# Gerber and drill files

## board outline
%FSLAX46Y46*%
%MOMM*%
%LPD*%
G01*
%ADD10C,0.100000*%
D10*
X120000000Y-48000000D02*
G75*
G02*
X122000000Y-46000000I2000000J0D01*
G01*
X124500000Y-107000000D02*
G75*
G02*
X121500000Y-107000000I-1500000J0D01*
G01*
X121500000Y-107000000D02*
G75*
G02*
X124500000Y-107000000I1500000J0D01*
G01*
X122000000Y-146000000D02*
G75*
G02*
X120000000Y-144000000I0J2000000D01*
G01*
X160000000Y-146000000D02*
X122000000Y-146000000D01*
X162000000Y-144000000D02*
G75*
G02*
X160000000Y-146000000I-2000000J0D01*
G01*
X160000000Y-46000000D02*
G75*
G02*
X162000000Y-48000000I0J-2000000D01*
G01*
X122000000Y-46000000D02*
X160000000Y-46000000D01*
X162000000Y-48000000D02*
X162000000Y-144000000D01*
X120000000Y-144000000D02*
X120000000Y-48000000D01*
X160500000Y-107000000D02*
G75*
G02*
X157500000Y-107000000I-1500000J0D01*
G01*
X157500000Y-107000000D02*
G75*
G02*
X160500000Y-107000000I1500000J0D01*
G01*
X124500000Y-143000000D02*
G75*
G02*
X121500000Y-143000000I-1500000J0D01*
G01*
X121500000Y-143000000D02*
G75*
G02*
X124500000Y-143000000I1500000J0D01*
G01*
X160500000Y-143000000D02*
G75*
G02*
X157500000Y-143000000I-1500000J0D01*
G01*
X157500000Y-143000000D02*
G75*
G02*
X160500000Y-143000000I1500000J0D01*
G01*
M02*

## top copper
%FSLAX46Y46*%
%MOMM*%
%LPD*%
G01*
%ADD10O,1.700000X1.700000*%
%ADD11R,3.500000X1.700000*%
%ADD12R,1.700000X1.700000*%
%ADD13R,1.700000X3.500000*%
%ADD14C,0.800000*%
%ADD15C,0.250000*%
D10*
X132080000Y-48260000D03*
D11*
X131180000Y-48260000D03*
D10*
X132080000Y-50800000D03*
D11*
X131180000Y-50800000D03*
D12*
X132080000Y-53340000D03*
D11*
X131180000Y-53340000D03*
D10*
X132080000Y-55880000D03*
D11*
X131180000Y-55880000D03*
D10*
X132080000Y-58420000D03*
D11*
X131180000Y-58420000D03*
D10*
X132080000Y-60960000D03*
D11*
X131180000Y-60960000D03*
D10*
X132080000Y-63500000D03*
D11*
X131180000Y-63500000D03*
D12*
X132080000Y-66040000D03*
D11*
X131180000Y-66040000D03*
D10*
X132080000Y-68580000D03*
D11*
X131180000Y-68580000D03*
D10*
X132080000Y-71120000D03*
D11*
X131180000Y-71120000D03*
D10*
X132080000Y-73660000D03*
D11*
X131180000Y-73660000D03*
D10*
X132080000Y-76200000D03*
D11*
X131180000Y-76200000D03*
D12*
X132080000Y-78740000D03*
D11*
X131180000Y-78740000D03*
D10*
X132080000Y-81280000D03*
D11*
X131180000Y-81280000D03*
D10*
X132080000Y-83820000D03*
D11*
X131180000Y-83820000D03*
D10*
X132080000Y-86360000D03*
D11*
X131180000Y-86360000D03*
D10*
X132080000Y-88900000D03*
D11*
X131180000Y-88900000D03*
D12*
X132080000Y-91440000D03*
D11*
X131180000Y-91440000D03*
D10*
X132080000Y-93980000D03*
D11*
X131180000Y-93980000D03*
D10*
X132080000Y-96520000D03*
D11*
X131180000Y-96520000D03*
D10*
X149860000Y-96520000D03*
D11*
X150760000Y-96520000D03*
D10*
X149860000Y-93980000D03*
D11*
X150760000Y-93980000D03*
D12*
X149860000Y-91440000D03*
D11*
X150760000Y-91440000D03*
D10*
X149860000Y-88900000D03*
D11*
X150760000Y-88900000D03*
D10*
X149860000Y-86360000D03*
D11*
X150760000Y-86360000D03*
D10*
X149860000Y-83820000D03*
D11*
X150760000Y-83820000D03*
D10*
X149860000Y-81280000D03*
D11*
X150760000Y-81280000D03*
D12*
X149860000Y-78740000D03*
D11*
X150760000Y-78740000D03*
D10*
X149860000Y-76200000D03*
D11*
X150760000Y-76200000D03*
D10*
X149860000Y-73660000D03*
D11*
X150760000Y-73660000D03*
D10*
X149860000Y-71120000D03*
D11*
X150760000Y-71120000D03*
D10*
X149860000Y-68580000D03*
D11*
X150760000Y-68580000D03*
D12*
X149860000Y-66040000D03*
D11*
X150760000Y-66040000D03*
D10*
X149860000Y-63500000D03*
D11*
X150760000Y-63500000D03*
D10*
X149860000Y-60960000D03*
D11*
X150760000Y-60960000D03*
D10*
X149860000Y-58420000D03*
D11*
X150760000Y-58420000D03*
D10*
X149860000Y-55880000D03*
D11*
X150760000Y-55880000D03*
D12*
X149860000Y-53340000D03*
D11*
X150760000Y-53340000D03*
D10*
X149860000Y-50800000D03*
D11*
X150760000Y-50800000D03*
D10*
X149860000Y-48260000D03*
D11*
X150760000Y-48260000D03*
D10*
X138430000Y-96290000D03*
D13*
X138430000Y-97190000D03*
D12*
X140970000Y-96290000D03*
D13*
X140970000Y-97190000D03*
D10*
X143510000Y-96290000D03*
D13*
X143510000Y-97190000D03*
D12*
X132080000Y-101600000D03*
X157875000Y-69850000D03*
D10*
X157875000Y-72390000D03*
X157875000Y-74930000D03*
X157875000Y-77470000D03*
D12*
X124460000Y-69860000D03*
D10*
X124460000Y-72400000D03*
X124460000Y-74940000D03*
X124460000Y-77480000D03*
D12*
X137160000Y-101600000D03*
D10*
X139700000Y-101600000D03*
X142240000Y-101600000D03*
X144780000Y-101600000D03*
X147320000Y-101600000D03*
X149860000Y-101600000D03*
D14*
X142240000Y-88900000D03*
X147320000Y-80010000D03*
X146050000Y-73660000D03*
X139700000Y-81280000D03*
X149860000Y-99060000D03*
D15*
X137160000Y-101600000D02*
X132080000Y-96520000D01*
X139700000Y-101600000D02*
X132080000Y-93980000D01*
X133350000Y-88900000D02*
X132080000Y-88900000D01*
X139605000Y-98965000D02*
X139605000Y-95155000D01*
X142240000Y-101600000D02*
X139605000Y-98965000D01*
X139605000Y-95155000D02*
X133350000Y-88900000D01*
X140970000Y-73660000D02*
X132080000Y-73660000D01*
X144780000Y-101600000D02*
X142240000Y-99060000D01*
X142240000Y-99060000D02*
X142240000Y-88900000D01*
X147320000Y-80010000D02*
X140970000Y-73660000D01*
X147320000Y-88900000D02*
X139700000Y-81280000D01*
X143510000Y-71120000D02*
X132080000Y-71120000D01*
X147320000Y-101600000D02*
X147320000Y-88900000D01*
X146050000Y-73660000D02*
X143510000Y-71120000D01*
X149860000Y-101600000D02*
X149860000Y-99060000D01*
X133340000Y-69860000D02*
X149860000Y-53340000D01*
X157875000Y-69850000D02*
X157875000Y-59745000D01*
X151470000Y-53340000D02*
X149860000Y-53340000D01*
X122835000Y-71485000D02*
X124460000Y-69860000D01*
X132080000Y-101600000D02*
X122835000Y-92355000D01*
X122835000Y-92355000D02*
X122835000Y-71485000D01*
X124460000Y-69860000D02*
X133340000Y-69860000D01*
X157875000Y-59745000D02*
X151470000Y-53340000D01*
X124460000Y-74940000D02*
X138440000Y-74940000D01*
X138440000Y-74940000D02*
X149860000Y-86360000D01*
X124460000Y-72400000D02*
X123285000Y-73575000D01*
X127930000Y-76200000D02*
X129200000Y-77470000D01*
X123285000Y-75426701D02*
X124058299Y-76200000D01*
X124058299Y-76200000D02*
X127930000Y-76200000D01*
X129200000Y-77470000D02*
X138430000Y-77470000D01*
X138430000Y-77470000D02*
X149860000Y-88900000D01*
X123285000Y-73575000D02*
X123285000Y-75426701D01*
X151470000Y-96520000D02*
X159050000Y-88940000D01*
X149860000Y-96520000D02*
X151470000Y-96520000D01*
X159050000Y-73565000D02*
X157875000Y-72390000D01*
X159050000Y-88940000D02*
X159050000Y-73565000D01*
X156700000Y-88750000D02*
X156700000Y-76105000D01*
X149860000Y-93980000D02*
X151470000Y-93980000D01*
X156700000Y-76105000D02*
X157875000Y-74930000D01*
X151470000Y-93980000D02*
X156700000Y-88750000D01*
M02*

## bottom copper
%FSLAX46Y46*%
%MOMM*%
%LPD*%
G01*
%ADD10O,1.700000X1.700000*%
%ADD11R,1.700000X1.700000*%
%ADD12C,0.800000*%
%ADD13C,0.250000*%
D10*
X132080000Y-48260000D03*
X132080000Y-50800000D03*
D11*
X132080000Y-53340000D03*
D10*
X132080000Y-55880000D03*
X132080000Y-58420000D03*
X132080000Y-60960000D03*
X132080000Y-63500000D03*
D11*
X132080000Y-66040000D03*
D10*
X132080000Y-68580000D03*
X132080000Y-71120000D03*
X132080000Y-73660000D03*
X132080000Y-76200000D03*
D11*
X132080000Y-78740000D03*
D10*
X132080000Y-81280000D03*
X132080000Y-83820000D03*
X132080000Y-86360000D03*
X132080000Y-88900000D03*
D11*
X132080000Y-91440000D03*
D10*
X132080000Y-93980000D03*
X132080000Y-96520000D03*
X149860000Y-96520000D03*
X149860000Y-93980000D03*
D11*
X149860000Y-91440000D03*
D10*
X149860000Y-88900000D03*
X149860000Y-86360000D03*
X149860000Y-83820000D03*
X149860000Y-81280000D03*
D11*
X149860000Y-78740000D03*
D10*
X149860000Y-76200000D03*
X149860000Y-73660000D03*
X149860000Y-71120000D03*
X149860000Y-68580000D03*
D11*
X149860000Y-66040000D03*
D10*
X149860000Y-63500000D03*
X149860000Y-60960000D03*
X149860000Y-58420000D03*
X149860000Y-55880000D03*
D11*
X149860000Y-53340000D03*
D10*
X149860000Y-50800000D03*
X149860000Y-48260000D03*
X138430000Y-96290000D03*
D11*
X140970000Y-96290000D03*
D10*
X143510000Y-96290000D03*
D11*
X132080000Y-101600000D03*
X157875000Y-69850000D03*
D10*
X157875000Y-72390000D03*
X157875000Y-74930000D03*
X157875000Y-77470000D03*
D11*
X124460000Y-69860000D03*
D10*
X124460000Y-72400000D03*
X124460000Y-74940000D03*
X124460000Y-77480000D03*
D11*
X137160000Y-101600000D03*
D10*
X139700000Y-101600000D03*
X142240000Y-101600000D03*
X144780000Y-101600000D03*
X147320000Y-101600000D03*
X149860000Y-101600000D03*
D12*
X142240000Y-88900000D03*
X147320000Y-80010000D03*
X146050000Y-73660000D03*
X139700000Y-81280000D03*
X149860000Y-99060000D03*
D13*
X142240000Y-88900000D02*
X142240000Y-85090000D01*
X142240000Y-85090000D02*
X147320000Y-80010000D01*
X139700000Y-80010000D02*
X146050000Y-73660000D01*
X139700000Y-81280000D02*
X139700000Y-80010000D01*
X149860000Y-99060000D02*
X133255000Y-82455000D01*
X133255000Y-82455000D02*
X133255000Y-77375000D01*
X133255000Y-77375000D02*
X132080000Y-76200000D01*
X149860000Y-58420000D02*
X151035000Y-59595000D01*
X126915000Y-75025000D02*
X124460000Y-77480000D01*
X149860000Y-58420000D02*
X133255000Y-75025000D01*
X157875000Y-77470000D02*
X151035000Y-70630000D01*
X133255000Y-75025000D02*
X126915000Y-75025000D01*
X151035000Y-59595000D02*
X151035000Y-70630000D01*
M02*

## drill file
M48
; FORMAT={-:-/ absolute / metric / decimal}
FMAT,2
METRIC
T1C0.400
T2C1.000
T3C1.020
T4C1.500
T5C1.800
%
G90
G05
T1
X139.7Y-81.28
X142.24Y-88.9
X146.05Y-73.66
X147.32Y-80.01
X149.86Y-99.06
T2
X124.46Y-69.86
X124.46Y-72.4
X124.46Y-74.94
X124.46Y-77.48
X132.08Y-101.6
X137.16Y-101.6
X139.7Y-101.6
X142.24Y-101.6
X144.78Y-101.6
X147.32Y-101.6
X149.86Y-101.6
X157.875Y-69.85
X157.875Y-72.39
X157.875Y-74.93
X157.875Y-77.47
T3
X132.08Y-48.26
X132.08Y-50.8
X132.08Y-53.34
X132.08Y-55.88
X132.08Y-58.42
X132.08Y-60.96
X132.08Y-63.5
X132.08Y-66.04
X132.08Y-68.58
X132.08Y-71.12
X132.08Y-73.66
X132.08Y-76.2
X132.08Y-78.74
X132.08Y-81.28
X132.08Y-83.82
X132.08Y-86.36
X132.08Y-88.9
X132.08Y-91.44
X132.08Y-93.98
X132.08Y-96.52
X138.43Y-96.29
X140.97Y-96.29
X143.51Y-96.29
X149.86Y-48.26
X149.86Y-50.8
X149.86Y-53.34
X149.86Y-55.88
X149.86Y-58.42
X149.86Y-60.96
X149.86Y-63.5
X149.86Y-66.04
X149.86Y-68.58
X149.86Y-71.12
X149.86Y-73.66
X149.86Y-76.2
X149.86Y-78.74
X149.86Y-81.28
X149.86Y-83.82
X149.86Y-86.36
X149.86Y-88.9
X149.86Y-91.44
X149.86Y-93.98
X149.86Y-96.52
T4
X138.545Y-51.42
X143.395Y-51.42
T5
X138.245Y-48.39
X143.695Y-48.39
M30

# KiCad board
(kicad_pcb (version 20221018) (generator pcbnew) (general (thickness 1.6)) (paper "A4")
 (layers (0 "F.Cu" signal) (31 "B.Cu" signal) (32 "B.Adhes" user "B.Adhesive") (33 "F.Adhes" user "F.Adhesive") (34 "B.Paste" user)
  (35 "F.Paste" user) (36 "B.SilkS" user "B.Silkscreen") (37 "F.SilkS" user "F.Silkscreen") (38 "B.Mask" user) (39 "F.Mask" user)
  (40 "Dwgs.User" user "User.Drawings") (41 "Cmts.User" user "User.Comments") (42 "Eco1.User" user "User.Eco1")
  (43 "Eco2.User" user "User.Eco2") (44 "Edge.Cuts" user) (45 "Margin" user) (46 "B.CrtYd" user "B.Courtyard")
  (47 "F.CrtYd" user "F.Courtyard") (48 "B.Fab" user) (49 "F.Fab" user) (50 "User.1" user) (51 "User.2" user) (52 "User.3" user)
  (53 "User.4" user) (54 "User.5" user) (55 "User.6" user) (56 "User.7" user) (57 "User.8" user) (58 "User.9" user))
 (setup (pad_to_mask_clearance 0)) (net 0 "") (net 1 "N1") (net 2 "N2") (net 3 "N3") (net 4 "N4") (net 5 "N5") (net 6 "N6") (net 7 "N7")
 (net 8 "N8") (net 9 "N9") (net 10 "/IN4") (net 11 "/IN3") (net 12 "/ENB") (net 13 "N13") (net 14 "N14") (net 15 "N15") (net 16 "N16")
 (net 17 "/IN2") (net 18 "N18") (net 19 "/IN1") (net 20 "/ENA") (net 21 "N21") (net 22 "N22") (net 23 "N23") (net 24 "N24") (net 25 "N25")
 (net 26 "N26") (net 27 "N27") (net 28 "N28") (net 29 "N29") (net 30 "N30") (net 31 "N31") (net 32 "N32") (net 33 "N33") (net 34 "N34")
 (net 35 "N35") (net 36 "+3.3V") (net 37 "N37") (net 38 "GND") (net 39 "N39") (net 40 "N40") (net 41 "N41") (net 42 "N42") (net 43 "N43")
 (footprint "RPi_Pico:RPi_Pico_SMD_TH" (layer "F.Cu") (at 140.97 72.39)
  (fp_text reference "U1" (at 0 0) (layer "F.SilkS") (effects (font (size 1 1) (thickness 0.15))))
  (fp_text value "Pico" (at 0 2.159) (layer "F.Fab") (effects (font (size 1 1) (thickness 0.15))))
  (pad "" np_thru_hole oval (at -2.725 -24) (size 1.8 1.8) (drill 1.8) (layers "*.Cu" "*.Mask"))
  (pad "" np_thru_hole oval (at -2.425 -20.97) (size 1.5 1.5) (drill 1.5) (layers "*.Cu" "*.Mask"))
  (pad "" np_thru_hole oval (at 2.425 -20.97) (size 1.5 1.5) (drill 1.5) (layers "*.Cu" "*.Mask"))
  (pad "" np_thru_hole oval (at 2.725 -24) (size 1.8 1.8) (drill 1.8) (layers "*.Cu" "*.Mask"))
  (pad "1" thru_hole oval (at -8.89 -24.13) (size 1.7 1.7) (drill 1.02) (layers "*.Cu" "*.Mask") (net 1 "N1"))
  (pad "1" smd rect (at -8.89 -24.13) (size 3.5 1.7) (drill (offset -0.9 0)) (layers "F.Cu" "F.Mask") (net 1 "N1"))
  (pad "2" thru_hole oval (at -8.89 -21.59) (size 1.7 1.7) (drill 1.02) (layers "*.Cu" "*.Mask") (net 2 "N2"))
  (pad "2" smd rect (at -8.89 -21.59) (size 3.5 1.7) (drill (offset -0.9 0)) (layers "F.Cu" "F.Mask") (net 2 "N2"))
  (pad "3" thru_hole rect (at -8.89 -19.05) (size 1.7 1.7) (drill 1.02) (layers "*.Cu" "*.Mask") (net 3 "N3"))
  (pad "3" smd rect (at -8.89 -19.05) (size 3.5 1.7) (drill (offset -0.9 0)) (layers "F.Cu" "F.Mask") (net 3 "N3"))
  (pad "4" thru_hole oval (at -8.89 -16.51) (size 1.7 1.7) (drill 1.02) (layers "*.Cu" "*.Mask") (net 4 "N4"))
  (pad "4" smd rect (at -8.89 -16.51) (size 3.5 1.7) (drill (offset -0.9 0)) (layers "F.Cu" "F.Mask") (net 4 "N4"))
  (pad "5" thru_hole oval (at -8.89 -13.97) (size 1.7 1.7) (drill 1.02) (layers "*.Cu" "*.Mask") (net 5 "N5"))
  (pad "5" smd rect (at -8.89 -13.97) (size 3.5 1.7) (drill (offset -0.9 0)) (layers "F.Cu" "F.Mask") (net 5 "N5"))
  (pad "6" thru_hole oval (at -8.89 -11.43) (size 1.7 1.7) (drill 1.02) (layers "*.Cu" "*.Mask") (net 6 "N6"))
  (pad "6" smd rect (at -8.89 -11.43) (size 3.5 1.7) (drill (offset -0.9 0)) (layers "F.Cu" "F.Mask") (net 6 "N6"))
  (pad "7" thru_hole oval (at -8.89 -8.89) (size 1.7 1.7) (drill 1.02) (layers "*.Cu" "*.Mask") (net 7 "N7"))
  (pad "7" smd rect (at -8.89 -8.89) (size 3.5 1.7) (drill (offset -0.9 0)) (layers "F.Cu" "F.Mask") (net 7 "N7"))
  (pad "8" thru_hole rect (at -8.89 -6.35) (size 1.7 1.7) (drill 1.02) (layers "*.Cu" "*.Mask") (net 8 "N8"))
  (pad "8" smd rect (at -8.89 -6.35) (size 3.5 1.7) (drill (offset -0.9 0)) (layers "F.Cu" "F.Mask") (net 8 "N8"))
  (pad "9" thru_hole oval (at -8.89 -3.81) (size 1.7 1.7) (drill 1.02) (layers "*.Cu" "*.Mask") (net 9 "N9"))
  (pad "9" smd rect (at -8.89 -3.81) (size 3.5 1.7) (drill (offset -0.9 0)) (layers "F.Cu" "F.Mask") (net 9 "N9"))
  (pad "10" thru_hole oval (at -8.89 -1.27) (size 1.7 1.7) (drill 1.02) (layers "*.Cu" "*.Mask") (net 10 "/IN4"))
  (pad "10" smd rect (at -8.89 -1.27) (size 3.5 1.7) (drill (offset -0.9 0)) (layers "F.Cu" "F.Mask") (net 10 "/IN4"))
  (pad "11" thru_hole oval (at -8.89 1.27) (size 1.7 1.7) (drill 1.02) (layers "*.Cu" "*.Mask") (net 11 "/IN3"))
  (pad "11" smd rect (at -8.89 1.27) (size 3.5 1.7) (drill (offset -0.9 0)) (layers "F.Cu" "F.Mask") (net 11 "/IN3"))
  (pad "12" thru_hole oval (at -8.89 3.81) (size 1.7 1.7) (drill 1.02) (layers "*.Cu" "*.Mask") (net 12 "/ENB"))
  (pad "12" smd rect (at -8.89 3.81) (size 3.5 1.7) (drill (offset -0.9 0)) (layers "F.Cu" "F.Mask") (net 12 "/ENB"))
  (pad "13" thru_hole rect (at -8.89 6.35) (size 1.7 1.7) (drill 1.02) (layers "*.Cu" "*.Mask") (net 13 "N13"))
  (pad "13" smd rect (at -8.89 6.35) (size 3.5 1.7) (drill (offset -0.9 0)) (layers "F.Cu" "F.Mask") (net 13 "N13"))
  (pad "14" thru_hole oval (at -8.89 8.89) (size 1.7 1.7) (drill 1.02) (layers "*.Cu" "*.Mask") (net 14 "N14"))
  (pad "14" smd rect (at -8.89 8.89) (size 3.5 1.7) (drill (offset -0.9 0)) (layers "F.Cu" "F.Mask") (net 14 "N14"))
  (pad "15" thru_hole oval (at -8.89 11.43) (size 1.7 1.7) (drill 1.02) (layers "*.Cu" "*.Mask") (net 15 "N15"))
  (pad "15" smd rect (at -8.89 11.43) (size 3.5 1.7) (drill (offset -0.9 0)) (layers "F.Cu" "F.Mask") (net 15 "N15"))
  (pad "16" thru_hole oval (at -8.89 13.97) (size 1.7 1.7) (drill 1.02) (layers "*.Cu" "*.Mask") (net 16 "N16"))
  (pad "16" smd rect (at -8.89 13.97) (size 3.5 1.7) (drill (offset -0.9 0)) (layers "F.Cu" "F.Mask") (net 16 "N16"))
  (pad "17" thru_hole oval (at -8.89 16.51) (size 1.7 1.7) (drill 1.02) (layers "*.Cu" "*.Mask") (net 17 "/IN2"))
  (pad "17" smd rect (at -8.89 16.51) (size 3.5 1.7) (drill (offset -0.9 0)) (layers "F.Cu" "F.Mask") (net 17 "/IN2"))
  (pad "18" thru_hole rect (at -8.89 19.05) (size 1.7 1.7) (drill 1.02) (layers "*.Cu" "*.Mask") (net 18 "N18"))
  (pad "18" smd rect (at -8.89 19.05) (size 3.5 1.7) (drill (offset -0.9 0)) (layers "F.Cu" "F.Mask") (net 18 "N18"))
  (pad "19" thru_hole oval (at -8.89 21.59) (size 1.7 1.7) (drill 1.02) (layers "*.Cu" "*.Mask") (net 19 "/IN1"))
  (pad "19" smd rect (at -8.89 21.59) (size 3.5 1.7) (drill (offset -0.9 0)) (layers "F.Cu" "F.Mask") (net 19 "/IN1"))
  (pad "20" thru_hole oval (at -8.89 24.13) (size 1.7 1.7) (drill 1.02) (layers "*.Cu" "*.Mask") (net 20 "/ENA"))
  (pad "20" smd rect (at -8.89 24.13) (size 3.5 1.7) (drill (offset -0.9 0)) (layers "F.Cu" "F.Mask") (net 20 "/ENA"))
  (pad "21" thru_hole oval (at 8.89 24.13) (size 1.7 1.7) (drill 1.02) (layers "*.Cu" "*.Mask") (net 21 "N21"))
  (pad "21" smd rect (at 8.89 24.13) (size 3.5 1.7) (drill (offset 0.9 0)) (layers "F.Cu" "F.Mask") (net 21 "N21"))
  (pad "22" thru_hole oval (at 8.89 21.59) (size 1.7 1.7) (drill 1.02) (layers "*.Cu" "*.Mask") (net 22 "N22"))
  (pad "22" smd rect (at 8.89 21.59) (size 3.5 1.7) (drill (offset 0.9 0)) (layers "F.Cu" "F.Mask") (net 22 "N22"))
  (pad "23" thru_hole rect (at 8.89 19.05) (size 1.7 1.7) (drill 1.02) (layers "*.Cu" "*.Mask") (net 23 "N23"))
  (pad "23" smd rect (at 8.89 19.05) (size 3.5 1.7) (drill (offset 0.9 0)) (layers "F.Cu" "F.Mask") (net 23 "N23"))
  (pad "24" thru_hole oval (at 8.89 16.51) (size 1.7 1.7) (drill 1.02) (layers "*.Cu" "*.Mask") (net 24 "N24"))
  (pad "24" smd rect (at 8.89 16.51) (size 3.5 1.7) (drill (offset 0.9 0)) (layers "F.Cu" "F.Mask") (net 24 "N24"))
  (pad "25" thru_hole oval (at 8.89 13.97) (size 1.7 1.7) (drill 1.02) (layers "*.Cu" "*.Mask") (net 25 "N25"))
  (pad "25" smd rect (at 8.89 13.97) (size 3.5 1.7) (drill (offset 0.9 0)) (layers "F.Cu" "F.Mask") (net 25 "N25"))
  (pad "26" thru_hole oval (at 8.89 11.43) (size 1.7 1.7) (drill 1.02) (layers "*.Cu" "*.Mask") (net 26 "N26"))
  (pad "26" smd rect (at 8.89 11.43) (size 3.5 1.7) (drill (offset 0.9 0)) (layers "F.Cu" "F.Mask") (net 26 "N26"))
  (pad "27" thru_hole oval (at 8.89 8.89) (size 1.7 1.7) (drill 1.02) (layers "*.Cu" "*.Mask") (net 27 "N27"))
  (pad "27" smd rect (at 8.89 8.89) (size 3.5 1.7) (drill (offset 0.9 0)) (layers "F.Cu" "F.Mask") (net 27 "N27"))
  (pad "28" thru_hole rect (at 8.89 6.35) (size 1.7 1.7) (drill 1.02) (layers "*.Cu" "*.Mask") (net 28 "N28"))
  (pad "28" smd rect (at 8.89 6.35) (size 3.5 1.7) (drill (offset 0.9 0)) (layers "F.Cu" "F.Mask") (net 28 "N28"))
  (pad "29" thru_hole oval (at 8.89 3.81) (size 1.7 1.7) (drill 1.02) (layers "*.Cu" "*.Mask") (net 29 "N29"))
  (pad "29" smd rect (at 8.89 3.81) (size 3.5 1.7) (drill (offset 0.9 0)) (layers "F.Cu" "F.Mask") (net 29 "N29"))
  (pad "30" thru_hole oval (at 8.89 1.27) (size 1.7 1.7) (drill 1.02) (layers "*.Cu" "*.Mask") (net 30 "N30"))
  (pad "30" smd rect (at 8.89 1.27) (size 3.5 1.7) (drill (offset 0.9 0)) (layers "F.Cu" "F.Mask") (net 30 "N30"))
  (pad "31" thru_hole oval (at 8.89 -1.27) (size 1.7 1.7) (drill 1.02) (layers "*.Cu" "*.Mask") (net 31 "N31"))
  (pad "31" smd rect (at 8.89 -1.27) (size 3.5 1.7) (drill (offset 0.9 0)) (layers "F.Cu" "F.Mask") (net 31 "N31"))
  (pad "32" thru_hole oval (at 8.89 -3.81) (size 1.7 1.7) (drill 1.02) (layers "*.Cu" "*.Mask") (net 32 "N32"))
  (pad "32" smd rect (at 8.89 -3.81) (size 3.5 1.7) (drill (offset 0.9 0)) (layers "F.Cu" "F.Mask") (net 32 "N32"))
  (pad "33" thru_hole rect (at 8.89 -6.35) (size 1.7 1.7) (drill 1.02) (layers "*.Cu" "*.Mask") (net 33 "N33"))
  (pad "33" smd rect (at 8.89 -6.35) (size 3.5 1.7) (drill (offset 0.9 0)) (layers "F.Cu" "F.Mask") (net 33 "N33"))
  (pad "34" thru_hole oval (at 8.89 -8.89) (size 1.7 1.7) (drill 1.02) (layers "*.Cu" "*.Mask") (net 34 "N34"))
  (pad "34" smd rect (at 8.89 -8.89) (size 3.5 1.7) (drill (offset 0.9 0)) (layers "F.Cu" "F.Mask") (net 34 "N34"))
  (pad "35" thru_hole oval (at 8.89 -11.43) (size 1.7 1.7) (drill 1.02) (layers "*.Cu" "*.Mask") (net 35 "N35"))
  (pad "35" smd rect (at 8.89 -11.43) (size 3.5 1.7) (drill (offset 0.9 0)) (layers "F.Cu" "F.Mask") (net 35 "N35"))
  (pad "36" thru_hole oval (at 8.89 -13.97) (size 1.7 1.7) (drill 1.02) (layers "*.Cu" "*.Mask") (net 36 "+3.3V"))
  (pad "36" smd rect (at 8.89 -13.97) (size 3.5 1.7) (drill (offset 0.9 0)) (layers "F.Cu" "F.Mask") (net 36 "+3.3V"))
  (pad "37" thru_hole oval (at 8.89 -16.51) (size 1.7 1.7) (drill 1.02) (layers "*.Cu" "*.Mask") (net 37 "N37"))
  (pad "37" smd rect (at 8.89 -16.51) (size 3.5 1.7) (drill (offset 0.9 0)) (layers "F.Cu" "F.Mask") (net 37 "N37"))
  (pad "38" thru_hole rect (at 8.89 -19.05) (size 1.7 1.7) (drill 1.02) (layers "*.Cu" "*.Mask") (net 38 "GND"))
  (pad "38" smd rect (at 8.89 -19.05) (size 3.5 1.7) (drill (offset 0.9 0)) (layers "F.Cu" "F.Mask") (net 38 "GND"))
  (pad "39" thru_hole oval (at 8.89 -21.59) (size 1.7 1.7) (drill 1.02) (layers "*.Cu" "*.Mask") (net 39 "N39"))
  (pad "39" smd rect (at 8.89 -21.59) (size 3.5 1.7) (drill (offset 0.9 0)) (layers "F.Cu" "F.Mask") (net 39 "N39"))
  (pad "40" thru_hole oval (at 8.89 -24.13) (size 1.7 1.7) (drill 1.02) (layers "*.Cu" "*.Mask") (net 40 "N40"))
  (pad "40" smd rect (at 8.89 -24.13) (size 3.5 1.7) (drill (offset 0.9 0)) (layers "F.Cu" "F.Mask") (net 40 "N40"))
  (pad "41" thru_hole oval (at -2.54 23.9) (size 1.7 1.7) (drill 1.02) (layers "*.Cu" "*.Mask") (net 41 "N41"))
  (pad "41" smd rect (at -2.54 23.9 90) (size 3.5 1.7) (drill (offset -0.9 0)) (layers "F.Cu" "F.Mask") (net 41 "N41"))
  (pad "42" thru_hole rect (at 0 23.9) (size 1.7 1.7) (drill 1.02) (layers "*.Cu" "*.Mask") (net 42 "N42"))
  (pad "42" smd rect (at 0 23.9 90) (size 3.5 1.7) (drill (offset -0.9 0)) (layers "F.Cu" "F.Mask") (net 42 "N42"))
  (pad "43" thru_hole oval (at 2.54 23.9) (size 1.7 1.7) (drill 1.02) (layers "*.Cu" "*.Mask") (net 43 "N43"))
  (pad "43" smd rect (at 2.54 23.9 90) (size 3.5 1.7) (drill (offset -0.9 0)) (layers "F.Cu" "F.Mask") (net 43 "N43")))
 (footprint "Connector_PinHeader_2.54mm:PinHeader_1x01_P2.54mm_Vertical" (layer "F.Cu") (at 132.08 101.6)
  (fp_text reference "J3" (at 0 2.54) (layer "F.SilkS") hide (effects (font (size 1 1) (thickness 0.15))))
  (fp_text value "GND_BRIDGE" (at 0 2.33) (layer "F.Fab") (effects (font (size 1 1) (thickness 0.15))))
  (pad "1" thru_hole rect (at 0 0) (size 1.7 1.7) (drill 1) (layers "*.Cu" "*.Mask") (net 38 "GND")))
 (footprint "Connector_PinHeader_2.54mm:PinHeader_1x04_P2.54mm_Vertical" (layer "F.Cu") (at 157.875 69.85)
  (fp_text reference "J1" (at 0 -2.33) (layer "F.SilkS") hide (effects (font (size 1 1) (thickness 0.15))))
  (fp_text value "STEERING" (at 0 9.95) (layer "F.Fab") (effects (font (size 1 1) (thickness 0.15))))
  (pad "1" thru_hole rect (at 0 0) (size 1.7 1.7) (drill 1) (layers "*.Cu" "*.Mask") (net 38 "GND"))
  (pad "2" thru_hole oval (at 0 2.54) (size 1.7 1.7) (drill 1) (layers "*.Cu" "*.Mask") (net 21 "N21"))
  (pad "3" thru_hole oval (at 0 5.08) (size 1.7 1.7) (drill 1) (layers "*.Cu" "*.Mask") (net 22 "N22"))
  (pad "4" thru_hole oval (at 0 7.62) (size 1.7 1.7) (drill 1) (layers "*.Cu" "*.Mask") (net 36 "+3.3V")))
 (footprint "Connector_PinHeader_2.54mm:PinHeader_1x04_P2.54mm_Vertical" (layer "F.Cu") (at 124.46 69.86)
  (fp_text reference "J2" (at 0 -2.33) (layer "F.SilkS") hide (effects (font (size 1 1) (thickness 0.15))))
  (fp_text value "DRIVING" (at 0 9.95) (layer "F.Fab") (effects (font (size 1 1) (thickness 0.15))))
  (pad "1" thru_hole rect (at 0 0) (size 1.7 1.7) (drill 1) (layers "*.Cu" "*.Mask") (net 38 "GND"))
  (pad "2" thru_hole oval (at 0 2.54) (size 1.7 1.7) (drill 1) (layers "*.Cu" "*.Mask") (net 24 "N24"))
  (pad "3" thru_hole oval (at 0 5.08) (size 1.7 1.7) (drill 1) (layers "*.Cu" "*.Mask") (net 25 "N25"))
  (pad "4" thru_hole oval (at 0 7.62) (size 1.7 1.7) (drill 1) (layers "*.Cu" "*.Mask") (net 36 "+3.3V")))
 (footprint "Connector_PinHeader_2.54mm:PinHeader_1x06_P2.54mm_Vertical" (layer "F.Cu") (at 137.16 101.6 90)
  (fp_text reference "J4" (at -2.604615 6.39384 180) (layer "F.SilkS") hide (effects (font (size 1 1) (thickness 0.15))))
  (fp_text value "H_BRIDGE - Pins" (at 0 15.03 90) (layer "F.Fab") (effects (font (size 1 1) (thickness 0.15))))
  (pad "1" thru_hole rect (at 0 0 90) (size 1.7 1.7) (drill 1) (layers "*.Cu" "*.Mask") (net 20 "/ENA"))
  (pad "2" thru_hole oval (at 0 2.54 90) (size 1.7 1.7) (drill 1) (layers "*.Cu" "*.Mask") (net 19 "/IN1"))
  (pad "3" thru_hole oval (at 0 5.08 90) (size 1.7 1.7) (drill 1) (layers "*.Cu" "*.Mask") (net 17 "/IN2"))
  (pad "4" thru_hole oval (at 0 7.62 90) (size 1.7 1.7) (drill 1) (layers "*.Cu" "*.Mask") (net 11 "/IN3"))
  (pad "5" thru_hole oval (at 0 10.16 90) (size 1.7 1.7) (drill 1) (layers "*.Cu" "*.Mask") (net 10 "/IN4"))
  (pad "6" thru_hole oval (at 0 12.7 90) (size 1.7 1.7) (drill 1) (layers "*.Cu" "*.Mask") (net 12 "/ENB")))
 (gr_arc (start 120 48) (mid 120.585786 46.585786) (end 122 46) (stroke (width 0.1) (type default)) (layer "Edge.Cuts"))
 (gr_circle (center 123 107) (end 124.5 107) (stroke (width 0.1) (type default)) (fill none) (layer "Edge.Cuts"))
 (gr_arc (start 122 146) (mid 120.585786 145.414214) (end 120 144) (stroke (width 0.1) (type default)) (layer "Edge.Cuts"))
 (gr_line (start 160 146) (end 122 146) (stroke (width 0.1) (type default)) (layer "Edge.Cuts"))
 (gr_arc (start 162 144) (mid 161.414214 145.414214) (end 160 146) (stroke (width 0.1) (type default)) (layer "Edge.Cuts"))
 (gr_arc (start 160 46) (mid 161.414214 46.585786) (end 162 48) (stroke (width 0.1) (type default)) (layer "Edge.Cuts"))
 (gr_line (start 122 46) (end 160 46) (stroke (width 0.1) (type default)) (layer "Edge.Cuts"))
 (gr_line (start 162 48) (end 162 144) (stroke (width 0.1) (type default)) (layer "Edge.Cuts"))
 (gr_line (start 120 144) (end 120 48) (stroke (width 0.1) (type default)) (layer "Edge.Cuts"))
 (gr_circle (center 159 107) (end 160.5 107) (stroke (width 0.1) (type default)) (fill none) (layer "Edge.Cuts"))
 (gr_circle (center 123 143) (end 124.5 143) (stroke (width 0.1) (type default)) (fill none) (layer "Edge.Cuts"))
 (gr_circle (center 159 143) (end 160.5 143) (stroke (width 0.1) (type default)) (fill none) (layer "Edge.Cuts"))
 (segment (start 137.16 101.6) (end 132.08 96.52) (width 0.25) (layer "F.Cu") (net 20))
 (segment (start 139.7 101.6) (end 132.08 93.98) (width 0.25) (layer "F.Cu") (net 19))
 (segment (start 133.35 88.9) (end 132.08 88.9) (width 0.25) (layer "F.Cu") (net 17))
 (segment (start 139.605 98.965) (end 139.605 95.155) (width 0.25) (layer "F.Cu") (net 17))
 (segment (start 142.24 101.6) (end 139.605 98.965) (width 0.25) (layer "F.Cu") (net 17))
 (segment (start 139.605 95.155) (end 133.35 88.9) (width 0.25) (layer "F.Cu") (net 17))
 (segment (start 140.97 73.66) (end 132.08 73.66) (width 0.25) (layer "F.Cu") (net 11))
 (segment (start 144.78 101.6) (end 142.24 99.06) (width 0.25) (layer "F.Cu") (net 11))
 (segment (start 142.24 99.06) (end 142.24 88.9) (width 0.25) (layer "F.Cu") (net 11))
 (segment (start 147.32 80.01) (end 140.97 73.66) (width 0.25) (layer "F.Cu") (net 11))
 (via (at 142.24 88.9) (size 0.8) (drill 0.4) (layers "F.Cu" "B.Cu") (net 11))
 (via (at 147.32 80.01) (size 0.8) (drill 0.4) (layers "F.Cu" "B.Cu") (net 11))
 (segment (start 142.24 88.9) (end 142.24 85.09) (width 0.25) (layer "B.Cu") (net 11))
 (segment (start 142.24 85.09) (end 147.32 80.01) (width 0.25) (layer "B.Cu") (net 11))
 (segment (start 147.32 88.9) (end 139.7 81.28) (width 0.25) (layer "F.Cu") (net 10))
 (segment (start 143.51 71.12) (end 132.08 71.12) (width 0.25) (layer "F.Cu") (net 10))
 (segment (start 147.32 101.6) (end 147.32 88.9) (width 0.25) (layer "F.Cu") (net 10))
 (segment (start 146.05 73.66) (end 143.51 71.12) (width 0.25) (layer "F.Cu") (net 10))
 (via (at 146.05 73.66) (size 0.8) (drill 0.4) (layers "F.Cu" "B.Cu") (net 10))
 (via (at 139.7 81.28) (size 0.8) (drill 0.4) (layers "F.Cu" "B.Cu") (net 10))
 (segment (start 139.7 80.01) (end 146.05 73.66) (width 0.25) (layer "B.Cu") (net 10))
 (segment (start 139.7 81.28) (end 139.7 80.01) (width 0.25) (layer "B.Cu") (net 10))
 (segment (start 149.86 101.6) (end 149.86 99.06) (width 0.25) (layer "F.Cu") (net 12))
 (via (at 149.86 99.06) (size 0.8) (drill 0.4) (layers "F.Cu" "B.Cu") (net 12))
 (segment (start 149.86 99.06) (end 133.255 82.455) (width 0.25) (layer "B.Cu") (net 12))
 (segment (start 133.255 82.455) (end 133.255 77.375) (width 0.25) (layer "B.Cu") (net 12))
 (segment (start 133.255 77.375) (end 132.08 76.2) (width 0.25) (layer "B.Cu") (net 12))
 (segment (start 133.34 69.86) (end 149.86 53.34) (width 0.25) (layer "F.Cu") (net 38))
 (segment (start 157.875 69.85) (end 157.875 59.745) (width 0.25) (layer "F.Cu") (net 38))
 (segment (start 151.47 53.34) (end 149.86 53.34) (width 0.25) (layer "F.Cu") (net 38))
 (segment (start 122.835 71.485) (end 124.46 69.86) (width 0.25) (layer "F.Cu") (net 38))
 (segment (start 132.08 101.6) (end 122.835 92.355) (width 0.25) (layer "F.Cu") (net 38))
 (segment (start 122.835 92.355) (end 122.835 71.485) (width 0.25) (layer "F.Cu") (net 38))
 (segment (start 124.46 69.86) (end 133.34 69.86) (width 0.25) (layer "F.Cu") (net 38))
 (segment (start 157.875 59.745) (end 151.47 53.34) (width 0.25) (layer "F.Cu") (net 38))
 (segment (start 124.46 74.94) (end 138.44 74.94) (width 0.25) (layer "F.Cu") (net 25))
 (segment (start 138.44 74.94) (end 149.86 86.36) (width 0.25) (layer "F.Cu") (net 25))
 (segment (start 149.86 58.42) (end 151.035 59.595) (width 0.25) (layer "B.Cu") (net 36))
 (segment (start 126.915 75.025) (end 124.46 77.48) (width 0.25) (layer "B.Cu") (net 36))
 (segment (start 149.86 58.42) (end 133.255 75.025) (width 0.25) (layer "B.Cu") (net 36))
 (segment (start 157.875 77.47) (end 151.035 70.63) (width 0.25) (layer "B.Cu") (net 36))
 (segment (start 133.255 75.025) (end 126.915 75.025) (width 0.25) (layer "B.Cu") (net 36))
 (segment (start 151.035 59.595) (end 151.035 70.63) (width 0.25) (layer "B.Cu") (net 36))
 (segment (start 124.46 72.4) (end 123.285 73.575) (width 0.25) (layer "F.Cu") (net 24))
 (segment (start 127.93 76.2) (end 129.2 77.47) (width 0.25) (layer "F.Cu") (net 24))
 (segment (start 123.285 75.426701) (end 124.058299 76.2) (width 0.25) (layer "F.Cu") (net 24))
 (segment (start 124.058299 76.2) (end 127.93 76.2) (width 0.25) (layer "F.Cu") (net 24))
 (segment (start 129.2 77.47) (end 138.43 77.47) (width 0.25) (layer "F.Cu") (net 24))
 (segment (start 138.43 77.47) (end 149.86 88.9) (width 0.25) (layer "F.Cu") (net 24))
 (segment (start 123.285 73.575) (end 123.285 75.426701) (width 0.25) (layer "F.Cu") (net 24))
 (segment (start 151.47 96.52) (end 159.05 88.94) (width 0.25) (layer "F.Cu") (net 21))
 (segment (start 149.86 96.52) (end 151.47 96.52) (width 0.25) (layer "F.Cu") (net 21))
 (segment (start 159.05 73.565) (end 157.875 72.39) (width 0.25) (layer "F.Cu") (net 21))
 (segment (start 159.05 88.94) (end 159.05 73.565) (width 0.25) (layer "F.Cu") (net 21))
 (segment (start 156.7 88.75) (end 156.7 76.105) (width 0.25) (layer "F.Cu") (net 22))
 (segment (start 149.86 93.98) (end 151.47 93.98) (width 0.25) (layer "F.Cu") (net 22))
 (segment (start 156.7 76.105) (end 157.875 74.93) (width 0.25) (layer "F.Cu") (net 22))
 (segment (start 151.47 93.98) (end 156.7 88.75) (width 0.25) (layer "F.Cu") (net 22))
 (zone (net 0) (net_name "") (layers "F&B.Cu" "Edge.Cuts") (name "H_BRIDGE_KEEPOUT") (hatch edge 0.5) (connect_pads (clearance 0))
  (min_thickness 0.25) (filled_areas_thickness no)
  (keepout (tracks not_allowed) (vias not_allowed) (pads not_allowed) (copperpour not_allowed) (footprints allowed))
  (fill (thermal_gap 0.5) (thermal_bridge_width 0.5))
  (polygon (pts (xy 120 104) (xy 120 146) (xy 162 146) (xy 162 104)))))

